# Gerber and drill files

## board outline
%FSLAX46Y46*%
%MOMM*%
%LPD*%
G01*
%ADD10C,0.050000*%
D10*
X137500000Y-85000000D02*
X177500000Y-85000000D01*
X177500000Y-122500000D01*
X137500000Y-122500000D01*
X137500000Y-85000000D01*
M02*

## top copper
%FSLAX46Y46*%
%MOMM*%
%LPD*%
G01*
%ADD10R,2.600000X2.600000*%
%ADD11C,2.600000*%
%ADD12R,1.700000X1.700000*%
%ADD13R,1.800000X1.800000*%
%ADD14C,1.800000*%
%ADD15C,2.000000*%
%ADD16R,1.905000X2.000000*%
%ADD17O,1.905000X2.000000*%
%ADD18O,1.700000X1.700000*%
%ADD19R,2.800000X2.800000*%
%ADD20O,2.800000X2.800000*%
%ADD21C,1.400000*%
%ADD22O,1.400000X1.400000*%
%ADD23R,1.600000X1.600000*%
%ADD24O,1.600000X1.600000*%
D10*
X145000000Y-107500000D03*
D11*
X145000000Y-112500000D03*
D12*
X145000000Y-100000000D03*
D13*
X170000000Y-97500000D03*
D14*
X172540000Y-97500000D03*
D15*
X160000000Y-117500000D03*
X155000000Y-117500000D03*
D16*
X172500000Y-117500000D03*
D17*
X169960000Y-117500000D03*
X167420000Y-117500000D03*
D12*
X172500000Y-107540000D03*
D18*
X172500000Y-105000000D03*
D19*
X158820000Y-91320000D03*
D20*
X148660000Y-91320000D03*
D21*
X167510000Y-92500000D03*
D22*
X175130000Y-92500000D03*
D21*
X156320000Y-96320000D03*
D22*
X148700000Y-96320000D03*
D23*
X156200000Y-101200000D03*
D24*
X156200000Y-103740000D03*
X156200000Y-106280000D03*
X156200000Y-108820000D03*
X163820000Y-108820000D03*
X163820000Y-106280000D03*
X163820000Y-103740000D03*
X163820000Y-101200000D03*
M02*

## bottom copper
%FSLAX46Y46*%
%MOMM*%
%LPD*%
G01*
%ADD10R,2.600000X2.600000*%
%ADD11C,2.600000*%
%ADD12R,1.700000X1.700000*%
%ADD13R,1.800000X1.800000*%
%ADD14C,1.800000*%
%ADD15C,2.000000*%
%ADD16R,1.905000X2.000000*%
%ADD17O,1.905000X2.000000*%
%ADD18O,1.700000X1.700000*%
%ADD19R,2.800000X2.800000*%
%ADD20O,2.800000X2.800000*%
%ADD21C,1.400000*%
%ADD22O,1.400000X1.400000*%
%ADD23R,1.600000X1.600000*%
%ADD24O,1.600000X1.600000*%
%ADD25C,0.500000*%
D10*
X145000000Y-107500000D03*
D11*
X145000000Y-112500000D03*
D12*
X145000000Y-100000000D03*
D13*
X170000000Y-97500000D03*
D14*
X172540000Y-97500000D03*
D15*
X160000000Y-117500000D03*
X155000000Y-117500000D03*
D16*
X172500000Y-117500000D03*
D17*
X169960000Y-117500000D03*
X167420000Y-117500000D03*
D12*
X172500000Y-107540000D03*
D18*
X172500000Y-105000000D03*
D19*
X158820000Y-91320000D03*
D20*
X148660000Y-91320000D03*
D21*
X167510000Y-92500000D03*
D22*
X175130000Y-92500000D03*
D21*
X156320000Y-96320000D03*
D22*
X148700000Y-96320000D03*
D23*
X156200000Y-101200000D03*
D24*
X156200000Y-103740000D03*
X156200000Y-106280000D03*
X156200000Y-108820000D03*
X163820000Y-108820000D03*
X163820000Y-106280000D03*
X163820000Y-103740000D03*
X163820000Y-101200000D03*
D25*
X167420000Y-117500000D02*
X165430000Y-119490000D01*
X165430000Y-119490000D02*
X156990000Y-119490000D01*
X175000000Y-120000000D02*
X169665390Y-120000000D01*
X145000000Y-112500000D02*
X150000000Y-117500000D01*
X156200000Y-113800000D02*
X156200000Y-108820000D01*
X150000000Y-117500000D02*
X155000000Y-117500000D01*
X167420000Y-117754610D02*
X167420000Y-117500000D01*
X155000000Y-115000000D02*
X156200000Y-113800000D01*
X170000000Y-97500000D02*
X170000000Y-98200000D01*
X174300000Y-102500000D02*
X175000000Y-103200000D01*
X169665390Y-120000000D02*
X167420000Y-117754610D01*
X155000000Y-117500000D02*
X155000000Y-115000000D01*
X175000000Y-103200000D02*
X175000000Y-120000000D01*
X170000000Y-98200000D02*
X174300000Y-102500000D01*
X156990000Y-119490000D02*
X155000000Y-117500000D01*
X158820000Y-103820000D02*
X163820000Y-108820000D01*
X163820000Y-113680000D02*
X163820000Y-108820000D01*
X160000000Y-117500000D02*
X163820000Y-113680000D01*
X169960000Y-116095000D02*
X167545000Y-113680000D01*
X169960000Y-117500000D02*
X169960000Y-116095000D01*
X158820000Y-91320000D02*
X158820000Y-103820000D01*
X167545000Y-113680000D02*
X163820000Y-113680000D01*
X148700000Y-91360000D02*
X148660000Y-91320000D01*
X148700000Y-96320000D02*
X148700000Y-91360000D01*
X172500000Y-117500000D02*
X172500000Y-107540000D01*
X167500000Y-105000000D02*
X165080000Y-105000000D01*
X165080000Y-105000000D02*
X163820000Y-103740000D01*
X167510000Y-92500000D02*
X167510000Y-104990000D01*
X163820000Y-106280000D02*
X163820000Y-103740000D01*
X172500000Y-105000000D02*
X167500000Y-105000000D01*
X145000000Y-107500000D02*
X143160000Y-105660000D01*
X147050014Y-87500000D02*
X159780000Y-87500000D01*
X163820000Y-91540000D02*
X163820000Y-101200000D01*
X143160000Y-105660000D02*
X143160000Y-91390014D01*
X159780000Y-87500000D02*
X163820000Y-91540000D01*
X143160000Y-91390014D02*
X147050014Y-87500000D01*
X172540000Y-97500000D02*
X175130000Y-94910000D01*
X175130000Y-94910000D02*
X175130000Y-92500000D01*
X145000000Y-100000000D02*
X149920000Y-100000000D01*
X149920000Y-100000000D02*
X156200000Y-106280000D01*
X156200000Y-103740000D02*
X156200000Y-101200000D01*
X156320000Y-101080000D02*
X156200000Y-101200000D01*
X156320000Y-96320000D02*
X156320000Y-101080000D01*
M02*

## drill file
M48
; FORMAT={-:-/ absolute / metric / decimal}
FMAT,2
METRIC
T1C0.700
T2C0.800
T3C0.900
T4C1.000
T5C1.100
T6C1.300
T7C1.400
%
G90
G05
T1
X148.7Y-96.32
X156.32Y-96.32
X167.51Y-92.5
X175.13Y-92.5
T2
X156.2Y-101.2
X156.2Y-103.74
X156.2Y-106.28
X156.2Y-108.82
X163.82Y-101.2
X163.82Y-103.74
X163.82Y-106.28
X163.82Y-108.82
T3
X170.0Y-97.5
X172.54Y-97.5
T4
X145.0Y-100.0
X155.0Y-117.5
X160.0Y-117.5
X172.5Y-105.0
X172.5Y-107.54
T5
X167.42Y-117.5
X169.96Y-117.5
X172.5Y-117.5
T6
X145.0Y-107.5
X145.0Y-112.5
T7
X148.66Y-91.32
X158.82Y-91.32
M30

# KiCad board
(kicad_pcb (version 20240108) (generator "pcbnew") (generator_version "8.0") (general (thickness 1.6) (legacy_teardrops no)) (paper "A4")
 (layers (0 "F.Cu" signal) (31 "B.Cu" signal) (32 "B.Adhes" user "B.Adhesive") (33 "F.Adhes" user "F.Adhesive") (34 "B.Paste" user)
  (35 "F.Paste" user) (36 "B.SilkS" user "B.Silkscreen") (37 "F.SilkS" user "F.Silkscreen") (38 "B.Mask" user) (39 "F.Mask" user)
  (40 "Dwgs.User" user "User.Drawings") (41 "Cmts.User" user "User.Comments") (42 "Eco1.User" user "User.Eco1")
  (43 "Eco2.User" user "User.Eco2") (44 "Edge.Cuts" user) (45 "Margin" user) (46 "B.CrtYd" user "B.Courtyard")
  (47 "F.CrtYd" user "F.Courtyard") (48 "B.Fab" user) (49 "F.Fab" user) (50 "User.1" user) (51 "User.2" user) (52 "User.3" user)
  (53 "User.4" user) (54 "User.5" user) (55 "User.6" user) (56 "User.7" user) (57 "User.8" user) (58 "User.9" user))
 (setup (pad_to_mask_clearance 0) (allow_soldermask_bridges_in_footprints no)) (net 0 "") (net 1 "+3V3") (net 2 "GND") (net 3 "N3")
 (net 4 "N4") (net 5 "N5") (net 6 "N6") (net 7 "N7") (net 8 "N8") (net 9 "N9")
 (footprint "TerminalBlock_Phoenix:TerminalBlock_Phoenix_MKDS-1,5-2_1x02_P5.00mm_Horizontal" (layer "F.Cu") (at 145 107.5 -90)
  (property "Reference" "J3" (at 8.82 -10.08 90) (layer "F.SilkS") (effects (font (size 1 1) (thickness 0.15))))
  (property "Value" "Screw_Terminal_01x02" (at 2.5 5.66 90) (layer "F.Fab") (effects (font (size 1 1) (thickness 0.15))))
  (pad "1" thru_hole rect (at 0 0 270) (size 2.6 2.6) (drill 1.3) (layers "*.Cu" "*.Mask") (remove_unused_layers no) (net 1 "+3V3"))
  (pad "2" thru_hole circle (at 5 0 270) (size 2.6 2.6) (drill 1.3) (layers "*.Cu" "*.Mask") (remove_unused_layers no) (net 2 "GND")))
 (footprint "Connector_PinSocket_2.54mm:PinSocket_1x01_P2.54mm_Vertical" (layer "F.Cu") (at 145 100)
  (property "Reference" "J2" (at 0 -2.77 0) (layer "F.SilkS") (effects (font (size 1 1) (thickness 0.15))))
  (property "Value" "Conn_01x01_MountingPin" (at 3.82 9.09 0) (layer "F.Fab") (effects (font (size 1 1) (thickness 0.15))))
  (pad "1" thru_hole rect (at 0 0) (size 1.7 1.7) (drill 1) (layers "*.Cu" "*.Mask") (remove_unused_layers no) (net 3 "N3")))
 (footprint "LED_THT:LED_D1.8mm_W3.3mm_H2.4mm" (layer "F.Cu") (at 170 97.5)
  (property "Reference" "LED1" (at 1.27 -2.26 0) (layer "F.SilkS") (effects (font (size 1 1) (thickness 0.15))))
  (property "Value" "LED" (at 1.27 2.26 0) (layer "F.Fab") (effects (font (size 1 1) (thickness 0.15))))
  (pad "1" thru_hole rect (at 0 0) (size 1.8 1.8) (drill 0.9) (layers "*.Cu" "*.Mask") (remove_unused_layers no) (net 2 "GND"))
  (pad "2" thru_hole circle (at 2.54 0) (size 1.8 1.8) (drill 0.9) (layers "*.Cu" "*.Mask") (remove_unused_layers no) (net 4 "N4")))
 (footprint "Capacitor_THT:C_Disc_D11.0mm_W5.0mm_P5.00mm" (layer "F.Cu") (at 160 117.5 180)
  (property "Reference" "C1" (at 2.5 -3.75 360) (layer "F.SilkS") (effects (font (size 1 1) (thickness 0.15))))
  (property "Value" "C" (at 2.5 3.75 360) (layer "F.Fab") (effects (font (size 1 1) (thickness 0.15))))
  (pad "1" thru_hole circle (at 0 0 180) (size 2 2) (drill 1) (layers "*.Cu" "*.Mask") (remove_unused_layers no) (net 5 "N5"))
  (pad "2" thru_hole circle (at 5 0 180) (size 2 2) (drill 1) (layers "*.Cu" "*.Mask") (remove_unused_layers no) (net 2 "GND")))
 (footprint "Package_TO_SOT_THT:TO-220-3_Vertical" (layer "F.Cu") (at 172.5 117.5 180)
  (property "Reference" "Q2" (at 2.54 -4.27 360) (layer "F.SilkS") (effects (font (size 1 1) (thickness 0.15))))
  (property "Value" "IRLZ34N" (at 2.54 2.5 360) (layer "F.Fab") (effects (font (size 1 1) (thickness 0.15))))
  (pad "1" thru_hole rect (at 0 0 180) (size 1.905 2) (drill 1.1) (layers "*.Cu" "*.Mask") (remove_unused_layers no) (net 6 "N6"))
  (pad "2" thru_hole oval (at 2.54 0 180) (size 1.905 2) (drill 1.1) (layers "*.Cu" "*.Mask") (remove_unused_layers no) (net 5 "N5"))
  (pad "3" thru_hole oval (at 5.08 0 180) (size 1.905 2) (drill 1.1) (layers "*.Cu" "*.Mask") (remove_unused_layers no) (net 2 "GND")))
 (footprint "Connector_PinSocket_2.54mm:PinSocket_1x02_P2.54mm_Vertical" (layer "F.Cu") (at 172.5 107.54 180)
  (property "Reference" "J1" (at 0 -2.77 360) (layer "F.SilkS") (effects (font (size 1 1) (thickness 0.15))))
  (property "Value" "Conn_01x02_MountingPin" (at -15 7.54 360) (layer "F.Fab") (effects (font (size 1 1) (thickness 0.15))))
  (pad "1" thru_hole rect (at 0 0 180) (size 1.7 1.7) (drill 1) (layers "*.Cu" "*.Mask") (remove_unused_layers no) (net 6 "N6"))
  (pad "2" thru_hole oval (at 0 2.54 180) (size 1.7 1.7) (drill 1) (layers "*.Cu" "*.Mask") (remove_unused_layers no) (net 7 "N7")))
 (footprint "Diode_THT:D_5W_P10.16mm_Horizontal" (layer "F.Cu") (at 158.82 91.32 180)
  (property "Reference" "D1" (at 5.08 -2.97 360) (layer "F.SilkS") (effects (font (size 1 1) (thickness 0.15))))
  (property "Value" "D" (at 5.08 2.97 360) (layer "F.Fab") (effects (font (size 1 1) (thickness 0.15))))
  (pad "1" thru_hole rect (at 0 0 180) (size 2.8 2.8) (drill 1.4) (layers "*.Cu" "*.Mask") (remove_unused_layers no) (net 5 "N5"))
  (pad "2" thru_hole oval (at 10.16 0 180) (size 2.8 2.8) (drill 1.4) (layers "*.Cu" "*.Mask") (remove_unused_layers no) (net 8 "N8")))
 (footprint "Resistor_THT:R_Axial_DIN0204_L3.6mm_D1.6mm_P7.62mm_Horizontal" (layer "F.Cu") (at 167.51 92.5)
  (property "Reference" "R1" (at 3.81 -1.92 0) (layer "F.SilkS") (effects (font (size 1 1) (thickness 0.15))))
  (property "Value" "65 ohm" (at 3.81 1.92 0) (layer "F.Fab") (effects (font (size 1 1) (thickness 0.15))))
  (pad "1" thru_hole circle (at 0 0) (size 1.4 1.4) (drill 0.7) (layers "*.Cu" "*.Mask") (remove_unused_layers no) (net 7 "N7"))
  (pad "2" thru_hole oval (at 7.62 0) (size 1.4 1.4) (drill 0.7) (layers "*.Cu" "*.Mask") (remove_unused_layers no) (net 4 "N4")))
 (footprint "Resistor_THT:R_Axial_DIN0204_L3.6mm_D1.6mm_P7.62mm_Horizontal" (layer "F.Cu") (at 156.32 96.32 180)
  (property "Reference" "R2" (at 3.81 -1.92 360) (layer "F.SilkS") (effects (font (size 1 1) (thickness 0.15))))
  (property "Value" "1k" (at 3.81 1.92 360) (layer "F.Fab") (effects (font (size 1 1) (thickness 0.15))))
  (pad "1" thru_hole circle (at 0 0 180) (size 1.4 1.4) (drill 0.7) (layers "*.Cu" "*.Mask") (remove_unused_layers no) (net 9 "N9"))
  (pad "2" thru_hole oval (at 7.62 0 180) (size 1.4 1.4) (drill 0.7) (layers "*.Cu" "*.Mask") (remove_unused_layers no) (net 8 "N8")))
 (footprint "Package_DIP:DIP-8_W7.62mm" (layer "F.Cu") (at 156.2 101.2)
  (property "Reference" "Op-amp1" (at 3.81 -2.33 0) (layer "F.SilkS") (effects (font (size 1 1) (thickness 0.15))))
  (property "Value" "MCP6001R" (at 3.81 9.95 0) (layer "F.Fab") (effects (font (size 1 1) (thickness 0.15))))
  (pad "1" thru_hole rect (at 0 0) (size 1.6 1.6) (drill 0.8) (layers "*.Cu" "*.Mask") (remove_unused_layers no) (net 9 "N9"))
  (pad "2" thru_hole oval (at 0 2.54) (size 1.6 1.6) (drill 0.8) (layers "*.Cu" "*.Mask") (remove_unused_layers no) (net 9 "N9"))
  (pad "3" thru_hole oval (at 0 5.08) (size 1.6 1.6) (drill 0.8) (layers "*.Cu" "*.Mask") (remove_unused_layers no) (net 3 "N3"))
  (pad "4" thru_hole oval (at 0 7.62) (size 1.6 1.6) (drill 0.8) (layers "*.Cu" "*.Mask") (remove_unused_layers no) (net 2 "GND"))
  (pad "5" thru_hole oval (at 7.62 7.62) (size 1.6 1.6) (drill 0.8) (layers "*.Cu" "*.Mask") (remove_unused_layers no) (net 5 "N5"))
  (pad "6" thru_hole oval (at 7.62 5.08) (size 1.6 1.6) (drill 0.8) (layers "*.Cu" "*.Mask") (remove_unused_layers no) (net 7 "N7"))
  (pad "7" thru_hole oval (at 7.62 2.54) (size 1.6 1.6) (drill 0.8) (layers "*.Cu" "*.Mask") (remove_unused_layers no) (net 7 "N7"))
  (pad "8" thru_hole oval (at 7.62 0) (size 1.6 1.6) (drill 0.8) (layers "*.Cu" "*.Mask") (remove_unused_layers no) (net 1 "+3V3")))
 (gr_rect (start 137.5 85) (end 177.5 122.5) (stroke (width 0.05) (type default)) (fill none) (layer "Edge.Cuts"))
 (segment (start 167.42 117.5) (end 165.43 119.49) (width 0.5) (layer "B.Cu") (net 2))
 (segment (start 165.43 119.49) (end 156.99 119.49) (width 0.5) (layer "B.Cu") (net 2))
 (segment (start 175 120) (end 169.66539 120) (width 0.5) (layer "B.Cu") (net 2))
 (segment (start 145 112.5) (end 150 117.5) (width 0.5) (layer "B.Cu") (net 2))
 (segment (start 156.2 113.8) (end 156.2 108.82) (width 0.5) (layer "B.Cu") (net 2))
 (segment (start 150 117.5) (end 155 117.5) (width 0.5) (layer "B.Cu") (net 2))
 (segment (start 167.42 117.75461) (end 167.42 117.5) (width 0.5) (layer "B.Cu") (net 2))
 (segment (start 155 115) (end 156.2 113.8) (width 0.5) (layer "B.Cu") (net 2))
 (segment (start 170 97.5) (end 170 98.2) (width 0.5) (layer "B.Cu") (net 2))
 (segment (start 174.3 102.5) (end 175 103.2) (width 0.5) (layer "B.Cu") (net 2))
 (segment (start 169.66539 120) (end 167.42 117.75461) (width 0.5) (layer "B.Cu") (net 2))
 (segment (start 155 117.5) (end 155 115) (width 0.5) (layer "B.Cu") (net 2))
 (segment (start 175 103.2) (end 175 120) (width 0.5) (layer "B.Cu") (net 2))
 (segment (start 170 98.2) (end 174.3 102.5) (width 0.5) (layer "B.Cu") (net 2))
 (segment (start 156.99 119.49) (end 155 117.5) (width 0.5) (layer "B.Cu") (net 2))
 (segment (start 158.82 103.82) (end 163.82 108.82) (width 0.5) (layer "B.Cu") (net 5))
 (segment (start 163.82 113.68) (end 163.82 108.82) (width 0.5) (layer "B.Cu") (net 5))
 (segment (start 160 117.5) (end 163.82 113.68) (width 0.5) (layer "B.Cu") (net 5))
 (segment (start 169.96 116.095) (end 167.545 113.68) (width 0.5) (layer "B.Cu") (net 5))
 (segment (start 169.96 117.5) (end 169.96 116.095) (width 0.5) (layer "B.Cu") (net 5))
 (segment (start 158.82 91.32) (end 158.82 103.82) (width 0.5) (layer "B.Cu") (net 5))
 (segment (start 167.545 113.68) (end 163.82 113.68) (width 0.5) (layer "B.Cu") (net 5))
 (segment (start 148.7 91.36) (end 148.66 91.32) (width 0.5) (layer "B.Cu") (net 8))
 (segment (start 148.7 96.32) (end 148.7 91.36) (width 0.5) (layer "B.Cu") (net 8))
 (segment (start 172.5 117.5) (end 172.5 107.54) (width 0.5) (layer "B.Cu") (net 6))
 (segment (start 167.5 105) (end 165.08 105) (width 0.5) (layer "B.Cu") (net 7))
 (segment (start 165.08 105) (end 163.82 103.74) (width 0.5) (layer "B.Cu") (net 7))
 (segment (start 167.51 92.5) (end 167.51 104.99) (width 0.5) (layer "B.Cu") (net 7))
 (segment (start 163.82 106.28) (end 163.82 103.74) (width 0.5) (layer "B.Cu") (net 7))
 (segment (start 172.5 105) (end 167.5 105) (width 0.5) (layer "B.Cu") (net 7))
 (segment (start 145 107.5) (end 143.16 105.66) (width 0.5) (layer "B.Cu") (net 1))
 (segment (start 147.050014 87.5) (end 159.78 87.5) (width 0.5) (layer "B.Cu") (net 1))
 (segment (start 163.82 91.54) (end 163.82 101.2) (width 0.5) (layer "B.Cu") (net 1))
 (segment (start 143.16 105.66) (end 143.16 91.390014) (width 0.5) (layer "B.Cu") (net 1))
 (segment (start 159.78 87.5) (end 163.82 91.54) (width 0.5) (layer "B.Cu") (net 1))
 (segment (start 143.16 91.390014) (end 147.050014 87.5) (width 0.5) (layer "B.Cu") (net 1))
 (segment (start 172.54 97.5) (end 175.13 94.91) (width 0.5) (layer "B.Cu") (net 4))
 (segment (start 175.13 94.91) (end 175.13 92.5) (width 0.5) (layer "B.Cu") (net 4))
 (segment (start 145 100) (end 149.92 100) (width 0.5) (layer "B.Cu") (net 3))
 (segment (start 149.92 100) (end 156.2 106.28) (width 0.5) (layer "B.Cu") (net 3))
 (segment (start 156.2 103.74) (end 156.2 101.2) (width 0.5) (layer "B.Cu") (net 9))
 (segment (start 156.32 101.08) (end 156.2 101.2) (width 0.5) (layer "B.Cu") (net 9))
 (segment (start 156.32 96.32) (end 156.32 101.08) (width 0.5) (layer "B.Cu") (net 9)))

